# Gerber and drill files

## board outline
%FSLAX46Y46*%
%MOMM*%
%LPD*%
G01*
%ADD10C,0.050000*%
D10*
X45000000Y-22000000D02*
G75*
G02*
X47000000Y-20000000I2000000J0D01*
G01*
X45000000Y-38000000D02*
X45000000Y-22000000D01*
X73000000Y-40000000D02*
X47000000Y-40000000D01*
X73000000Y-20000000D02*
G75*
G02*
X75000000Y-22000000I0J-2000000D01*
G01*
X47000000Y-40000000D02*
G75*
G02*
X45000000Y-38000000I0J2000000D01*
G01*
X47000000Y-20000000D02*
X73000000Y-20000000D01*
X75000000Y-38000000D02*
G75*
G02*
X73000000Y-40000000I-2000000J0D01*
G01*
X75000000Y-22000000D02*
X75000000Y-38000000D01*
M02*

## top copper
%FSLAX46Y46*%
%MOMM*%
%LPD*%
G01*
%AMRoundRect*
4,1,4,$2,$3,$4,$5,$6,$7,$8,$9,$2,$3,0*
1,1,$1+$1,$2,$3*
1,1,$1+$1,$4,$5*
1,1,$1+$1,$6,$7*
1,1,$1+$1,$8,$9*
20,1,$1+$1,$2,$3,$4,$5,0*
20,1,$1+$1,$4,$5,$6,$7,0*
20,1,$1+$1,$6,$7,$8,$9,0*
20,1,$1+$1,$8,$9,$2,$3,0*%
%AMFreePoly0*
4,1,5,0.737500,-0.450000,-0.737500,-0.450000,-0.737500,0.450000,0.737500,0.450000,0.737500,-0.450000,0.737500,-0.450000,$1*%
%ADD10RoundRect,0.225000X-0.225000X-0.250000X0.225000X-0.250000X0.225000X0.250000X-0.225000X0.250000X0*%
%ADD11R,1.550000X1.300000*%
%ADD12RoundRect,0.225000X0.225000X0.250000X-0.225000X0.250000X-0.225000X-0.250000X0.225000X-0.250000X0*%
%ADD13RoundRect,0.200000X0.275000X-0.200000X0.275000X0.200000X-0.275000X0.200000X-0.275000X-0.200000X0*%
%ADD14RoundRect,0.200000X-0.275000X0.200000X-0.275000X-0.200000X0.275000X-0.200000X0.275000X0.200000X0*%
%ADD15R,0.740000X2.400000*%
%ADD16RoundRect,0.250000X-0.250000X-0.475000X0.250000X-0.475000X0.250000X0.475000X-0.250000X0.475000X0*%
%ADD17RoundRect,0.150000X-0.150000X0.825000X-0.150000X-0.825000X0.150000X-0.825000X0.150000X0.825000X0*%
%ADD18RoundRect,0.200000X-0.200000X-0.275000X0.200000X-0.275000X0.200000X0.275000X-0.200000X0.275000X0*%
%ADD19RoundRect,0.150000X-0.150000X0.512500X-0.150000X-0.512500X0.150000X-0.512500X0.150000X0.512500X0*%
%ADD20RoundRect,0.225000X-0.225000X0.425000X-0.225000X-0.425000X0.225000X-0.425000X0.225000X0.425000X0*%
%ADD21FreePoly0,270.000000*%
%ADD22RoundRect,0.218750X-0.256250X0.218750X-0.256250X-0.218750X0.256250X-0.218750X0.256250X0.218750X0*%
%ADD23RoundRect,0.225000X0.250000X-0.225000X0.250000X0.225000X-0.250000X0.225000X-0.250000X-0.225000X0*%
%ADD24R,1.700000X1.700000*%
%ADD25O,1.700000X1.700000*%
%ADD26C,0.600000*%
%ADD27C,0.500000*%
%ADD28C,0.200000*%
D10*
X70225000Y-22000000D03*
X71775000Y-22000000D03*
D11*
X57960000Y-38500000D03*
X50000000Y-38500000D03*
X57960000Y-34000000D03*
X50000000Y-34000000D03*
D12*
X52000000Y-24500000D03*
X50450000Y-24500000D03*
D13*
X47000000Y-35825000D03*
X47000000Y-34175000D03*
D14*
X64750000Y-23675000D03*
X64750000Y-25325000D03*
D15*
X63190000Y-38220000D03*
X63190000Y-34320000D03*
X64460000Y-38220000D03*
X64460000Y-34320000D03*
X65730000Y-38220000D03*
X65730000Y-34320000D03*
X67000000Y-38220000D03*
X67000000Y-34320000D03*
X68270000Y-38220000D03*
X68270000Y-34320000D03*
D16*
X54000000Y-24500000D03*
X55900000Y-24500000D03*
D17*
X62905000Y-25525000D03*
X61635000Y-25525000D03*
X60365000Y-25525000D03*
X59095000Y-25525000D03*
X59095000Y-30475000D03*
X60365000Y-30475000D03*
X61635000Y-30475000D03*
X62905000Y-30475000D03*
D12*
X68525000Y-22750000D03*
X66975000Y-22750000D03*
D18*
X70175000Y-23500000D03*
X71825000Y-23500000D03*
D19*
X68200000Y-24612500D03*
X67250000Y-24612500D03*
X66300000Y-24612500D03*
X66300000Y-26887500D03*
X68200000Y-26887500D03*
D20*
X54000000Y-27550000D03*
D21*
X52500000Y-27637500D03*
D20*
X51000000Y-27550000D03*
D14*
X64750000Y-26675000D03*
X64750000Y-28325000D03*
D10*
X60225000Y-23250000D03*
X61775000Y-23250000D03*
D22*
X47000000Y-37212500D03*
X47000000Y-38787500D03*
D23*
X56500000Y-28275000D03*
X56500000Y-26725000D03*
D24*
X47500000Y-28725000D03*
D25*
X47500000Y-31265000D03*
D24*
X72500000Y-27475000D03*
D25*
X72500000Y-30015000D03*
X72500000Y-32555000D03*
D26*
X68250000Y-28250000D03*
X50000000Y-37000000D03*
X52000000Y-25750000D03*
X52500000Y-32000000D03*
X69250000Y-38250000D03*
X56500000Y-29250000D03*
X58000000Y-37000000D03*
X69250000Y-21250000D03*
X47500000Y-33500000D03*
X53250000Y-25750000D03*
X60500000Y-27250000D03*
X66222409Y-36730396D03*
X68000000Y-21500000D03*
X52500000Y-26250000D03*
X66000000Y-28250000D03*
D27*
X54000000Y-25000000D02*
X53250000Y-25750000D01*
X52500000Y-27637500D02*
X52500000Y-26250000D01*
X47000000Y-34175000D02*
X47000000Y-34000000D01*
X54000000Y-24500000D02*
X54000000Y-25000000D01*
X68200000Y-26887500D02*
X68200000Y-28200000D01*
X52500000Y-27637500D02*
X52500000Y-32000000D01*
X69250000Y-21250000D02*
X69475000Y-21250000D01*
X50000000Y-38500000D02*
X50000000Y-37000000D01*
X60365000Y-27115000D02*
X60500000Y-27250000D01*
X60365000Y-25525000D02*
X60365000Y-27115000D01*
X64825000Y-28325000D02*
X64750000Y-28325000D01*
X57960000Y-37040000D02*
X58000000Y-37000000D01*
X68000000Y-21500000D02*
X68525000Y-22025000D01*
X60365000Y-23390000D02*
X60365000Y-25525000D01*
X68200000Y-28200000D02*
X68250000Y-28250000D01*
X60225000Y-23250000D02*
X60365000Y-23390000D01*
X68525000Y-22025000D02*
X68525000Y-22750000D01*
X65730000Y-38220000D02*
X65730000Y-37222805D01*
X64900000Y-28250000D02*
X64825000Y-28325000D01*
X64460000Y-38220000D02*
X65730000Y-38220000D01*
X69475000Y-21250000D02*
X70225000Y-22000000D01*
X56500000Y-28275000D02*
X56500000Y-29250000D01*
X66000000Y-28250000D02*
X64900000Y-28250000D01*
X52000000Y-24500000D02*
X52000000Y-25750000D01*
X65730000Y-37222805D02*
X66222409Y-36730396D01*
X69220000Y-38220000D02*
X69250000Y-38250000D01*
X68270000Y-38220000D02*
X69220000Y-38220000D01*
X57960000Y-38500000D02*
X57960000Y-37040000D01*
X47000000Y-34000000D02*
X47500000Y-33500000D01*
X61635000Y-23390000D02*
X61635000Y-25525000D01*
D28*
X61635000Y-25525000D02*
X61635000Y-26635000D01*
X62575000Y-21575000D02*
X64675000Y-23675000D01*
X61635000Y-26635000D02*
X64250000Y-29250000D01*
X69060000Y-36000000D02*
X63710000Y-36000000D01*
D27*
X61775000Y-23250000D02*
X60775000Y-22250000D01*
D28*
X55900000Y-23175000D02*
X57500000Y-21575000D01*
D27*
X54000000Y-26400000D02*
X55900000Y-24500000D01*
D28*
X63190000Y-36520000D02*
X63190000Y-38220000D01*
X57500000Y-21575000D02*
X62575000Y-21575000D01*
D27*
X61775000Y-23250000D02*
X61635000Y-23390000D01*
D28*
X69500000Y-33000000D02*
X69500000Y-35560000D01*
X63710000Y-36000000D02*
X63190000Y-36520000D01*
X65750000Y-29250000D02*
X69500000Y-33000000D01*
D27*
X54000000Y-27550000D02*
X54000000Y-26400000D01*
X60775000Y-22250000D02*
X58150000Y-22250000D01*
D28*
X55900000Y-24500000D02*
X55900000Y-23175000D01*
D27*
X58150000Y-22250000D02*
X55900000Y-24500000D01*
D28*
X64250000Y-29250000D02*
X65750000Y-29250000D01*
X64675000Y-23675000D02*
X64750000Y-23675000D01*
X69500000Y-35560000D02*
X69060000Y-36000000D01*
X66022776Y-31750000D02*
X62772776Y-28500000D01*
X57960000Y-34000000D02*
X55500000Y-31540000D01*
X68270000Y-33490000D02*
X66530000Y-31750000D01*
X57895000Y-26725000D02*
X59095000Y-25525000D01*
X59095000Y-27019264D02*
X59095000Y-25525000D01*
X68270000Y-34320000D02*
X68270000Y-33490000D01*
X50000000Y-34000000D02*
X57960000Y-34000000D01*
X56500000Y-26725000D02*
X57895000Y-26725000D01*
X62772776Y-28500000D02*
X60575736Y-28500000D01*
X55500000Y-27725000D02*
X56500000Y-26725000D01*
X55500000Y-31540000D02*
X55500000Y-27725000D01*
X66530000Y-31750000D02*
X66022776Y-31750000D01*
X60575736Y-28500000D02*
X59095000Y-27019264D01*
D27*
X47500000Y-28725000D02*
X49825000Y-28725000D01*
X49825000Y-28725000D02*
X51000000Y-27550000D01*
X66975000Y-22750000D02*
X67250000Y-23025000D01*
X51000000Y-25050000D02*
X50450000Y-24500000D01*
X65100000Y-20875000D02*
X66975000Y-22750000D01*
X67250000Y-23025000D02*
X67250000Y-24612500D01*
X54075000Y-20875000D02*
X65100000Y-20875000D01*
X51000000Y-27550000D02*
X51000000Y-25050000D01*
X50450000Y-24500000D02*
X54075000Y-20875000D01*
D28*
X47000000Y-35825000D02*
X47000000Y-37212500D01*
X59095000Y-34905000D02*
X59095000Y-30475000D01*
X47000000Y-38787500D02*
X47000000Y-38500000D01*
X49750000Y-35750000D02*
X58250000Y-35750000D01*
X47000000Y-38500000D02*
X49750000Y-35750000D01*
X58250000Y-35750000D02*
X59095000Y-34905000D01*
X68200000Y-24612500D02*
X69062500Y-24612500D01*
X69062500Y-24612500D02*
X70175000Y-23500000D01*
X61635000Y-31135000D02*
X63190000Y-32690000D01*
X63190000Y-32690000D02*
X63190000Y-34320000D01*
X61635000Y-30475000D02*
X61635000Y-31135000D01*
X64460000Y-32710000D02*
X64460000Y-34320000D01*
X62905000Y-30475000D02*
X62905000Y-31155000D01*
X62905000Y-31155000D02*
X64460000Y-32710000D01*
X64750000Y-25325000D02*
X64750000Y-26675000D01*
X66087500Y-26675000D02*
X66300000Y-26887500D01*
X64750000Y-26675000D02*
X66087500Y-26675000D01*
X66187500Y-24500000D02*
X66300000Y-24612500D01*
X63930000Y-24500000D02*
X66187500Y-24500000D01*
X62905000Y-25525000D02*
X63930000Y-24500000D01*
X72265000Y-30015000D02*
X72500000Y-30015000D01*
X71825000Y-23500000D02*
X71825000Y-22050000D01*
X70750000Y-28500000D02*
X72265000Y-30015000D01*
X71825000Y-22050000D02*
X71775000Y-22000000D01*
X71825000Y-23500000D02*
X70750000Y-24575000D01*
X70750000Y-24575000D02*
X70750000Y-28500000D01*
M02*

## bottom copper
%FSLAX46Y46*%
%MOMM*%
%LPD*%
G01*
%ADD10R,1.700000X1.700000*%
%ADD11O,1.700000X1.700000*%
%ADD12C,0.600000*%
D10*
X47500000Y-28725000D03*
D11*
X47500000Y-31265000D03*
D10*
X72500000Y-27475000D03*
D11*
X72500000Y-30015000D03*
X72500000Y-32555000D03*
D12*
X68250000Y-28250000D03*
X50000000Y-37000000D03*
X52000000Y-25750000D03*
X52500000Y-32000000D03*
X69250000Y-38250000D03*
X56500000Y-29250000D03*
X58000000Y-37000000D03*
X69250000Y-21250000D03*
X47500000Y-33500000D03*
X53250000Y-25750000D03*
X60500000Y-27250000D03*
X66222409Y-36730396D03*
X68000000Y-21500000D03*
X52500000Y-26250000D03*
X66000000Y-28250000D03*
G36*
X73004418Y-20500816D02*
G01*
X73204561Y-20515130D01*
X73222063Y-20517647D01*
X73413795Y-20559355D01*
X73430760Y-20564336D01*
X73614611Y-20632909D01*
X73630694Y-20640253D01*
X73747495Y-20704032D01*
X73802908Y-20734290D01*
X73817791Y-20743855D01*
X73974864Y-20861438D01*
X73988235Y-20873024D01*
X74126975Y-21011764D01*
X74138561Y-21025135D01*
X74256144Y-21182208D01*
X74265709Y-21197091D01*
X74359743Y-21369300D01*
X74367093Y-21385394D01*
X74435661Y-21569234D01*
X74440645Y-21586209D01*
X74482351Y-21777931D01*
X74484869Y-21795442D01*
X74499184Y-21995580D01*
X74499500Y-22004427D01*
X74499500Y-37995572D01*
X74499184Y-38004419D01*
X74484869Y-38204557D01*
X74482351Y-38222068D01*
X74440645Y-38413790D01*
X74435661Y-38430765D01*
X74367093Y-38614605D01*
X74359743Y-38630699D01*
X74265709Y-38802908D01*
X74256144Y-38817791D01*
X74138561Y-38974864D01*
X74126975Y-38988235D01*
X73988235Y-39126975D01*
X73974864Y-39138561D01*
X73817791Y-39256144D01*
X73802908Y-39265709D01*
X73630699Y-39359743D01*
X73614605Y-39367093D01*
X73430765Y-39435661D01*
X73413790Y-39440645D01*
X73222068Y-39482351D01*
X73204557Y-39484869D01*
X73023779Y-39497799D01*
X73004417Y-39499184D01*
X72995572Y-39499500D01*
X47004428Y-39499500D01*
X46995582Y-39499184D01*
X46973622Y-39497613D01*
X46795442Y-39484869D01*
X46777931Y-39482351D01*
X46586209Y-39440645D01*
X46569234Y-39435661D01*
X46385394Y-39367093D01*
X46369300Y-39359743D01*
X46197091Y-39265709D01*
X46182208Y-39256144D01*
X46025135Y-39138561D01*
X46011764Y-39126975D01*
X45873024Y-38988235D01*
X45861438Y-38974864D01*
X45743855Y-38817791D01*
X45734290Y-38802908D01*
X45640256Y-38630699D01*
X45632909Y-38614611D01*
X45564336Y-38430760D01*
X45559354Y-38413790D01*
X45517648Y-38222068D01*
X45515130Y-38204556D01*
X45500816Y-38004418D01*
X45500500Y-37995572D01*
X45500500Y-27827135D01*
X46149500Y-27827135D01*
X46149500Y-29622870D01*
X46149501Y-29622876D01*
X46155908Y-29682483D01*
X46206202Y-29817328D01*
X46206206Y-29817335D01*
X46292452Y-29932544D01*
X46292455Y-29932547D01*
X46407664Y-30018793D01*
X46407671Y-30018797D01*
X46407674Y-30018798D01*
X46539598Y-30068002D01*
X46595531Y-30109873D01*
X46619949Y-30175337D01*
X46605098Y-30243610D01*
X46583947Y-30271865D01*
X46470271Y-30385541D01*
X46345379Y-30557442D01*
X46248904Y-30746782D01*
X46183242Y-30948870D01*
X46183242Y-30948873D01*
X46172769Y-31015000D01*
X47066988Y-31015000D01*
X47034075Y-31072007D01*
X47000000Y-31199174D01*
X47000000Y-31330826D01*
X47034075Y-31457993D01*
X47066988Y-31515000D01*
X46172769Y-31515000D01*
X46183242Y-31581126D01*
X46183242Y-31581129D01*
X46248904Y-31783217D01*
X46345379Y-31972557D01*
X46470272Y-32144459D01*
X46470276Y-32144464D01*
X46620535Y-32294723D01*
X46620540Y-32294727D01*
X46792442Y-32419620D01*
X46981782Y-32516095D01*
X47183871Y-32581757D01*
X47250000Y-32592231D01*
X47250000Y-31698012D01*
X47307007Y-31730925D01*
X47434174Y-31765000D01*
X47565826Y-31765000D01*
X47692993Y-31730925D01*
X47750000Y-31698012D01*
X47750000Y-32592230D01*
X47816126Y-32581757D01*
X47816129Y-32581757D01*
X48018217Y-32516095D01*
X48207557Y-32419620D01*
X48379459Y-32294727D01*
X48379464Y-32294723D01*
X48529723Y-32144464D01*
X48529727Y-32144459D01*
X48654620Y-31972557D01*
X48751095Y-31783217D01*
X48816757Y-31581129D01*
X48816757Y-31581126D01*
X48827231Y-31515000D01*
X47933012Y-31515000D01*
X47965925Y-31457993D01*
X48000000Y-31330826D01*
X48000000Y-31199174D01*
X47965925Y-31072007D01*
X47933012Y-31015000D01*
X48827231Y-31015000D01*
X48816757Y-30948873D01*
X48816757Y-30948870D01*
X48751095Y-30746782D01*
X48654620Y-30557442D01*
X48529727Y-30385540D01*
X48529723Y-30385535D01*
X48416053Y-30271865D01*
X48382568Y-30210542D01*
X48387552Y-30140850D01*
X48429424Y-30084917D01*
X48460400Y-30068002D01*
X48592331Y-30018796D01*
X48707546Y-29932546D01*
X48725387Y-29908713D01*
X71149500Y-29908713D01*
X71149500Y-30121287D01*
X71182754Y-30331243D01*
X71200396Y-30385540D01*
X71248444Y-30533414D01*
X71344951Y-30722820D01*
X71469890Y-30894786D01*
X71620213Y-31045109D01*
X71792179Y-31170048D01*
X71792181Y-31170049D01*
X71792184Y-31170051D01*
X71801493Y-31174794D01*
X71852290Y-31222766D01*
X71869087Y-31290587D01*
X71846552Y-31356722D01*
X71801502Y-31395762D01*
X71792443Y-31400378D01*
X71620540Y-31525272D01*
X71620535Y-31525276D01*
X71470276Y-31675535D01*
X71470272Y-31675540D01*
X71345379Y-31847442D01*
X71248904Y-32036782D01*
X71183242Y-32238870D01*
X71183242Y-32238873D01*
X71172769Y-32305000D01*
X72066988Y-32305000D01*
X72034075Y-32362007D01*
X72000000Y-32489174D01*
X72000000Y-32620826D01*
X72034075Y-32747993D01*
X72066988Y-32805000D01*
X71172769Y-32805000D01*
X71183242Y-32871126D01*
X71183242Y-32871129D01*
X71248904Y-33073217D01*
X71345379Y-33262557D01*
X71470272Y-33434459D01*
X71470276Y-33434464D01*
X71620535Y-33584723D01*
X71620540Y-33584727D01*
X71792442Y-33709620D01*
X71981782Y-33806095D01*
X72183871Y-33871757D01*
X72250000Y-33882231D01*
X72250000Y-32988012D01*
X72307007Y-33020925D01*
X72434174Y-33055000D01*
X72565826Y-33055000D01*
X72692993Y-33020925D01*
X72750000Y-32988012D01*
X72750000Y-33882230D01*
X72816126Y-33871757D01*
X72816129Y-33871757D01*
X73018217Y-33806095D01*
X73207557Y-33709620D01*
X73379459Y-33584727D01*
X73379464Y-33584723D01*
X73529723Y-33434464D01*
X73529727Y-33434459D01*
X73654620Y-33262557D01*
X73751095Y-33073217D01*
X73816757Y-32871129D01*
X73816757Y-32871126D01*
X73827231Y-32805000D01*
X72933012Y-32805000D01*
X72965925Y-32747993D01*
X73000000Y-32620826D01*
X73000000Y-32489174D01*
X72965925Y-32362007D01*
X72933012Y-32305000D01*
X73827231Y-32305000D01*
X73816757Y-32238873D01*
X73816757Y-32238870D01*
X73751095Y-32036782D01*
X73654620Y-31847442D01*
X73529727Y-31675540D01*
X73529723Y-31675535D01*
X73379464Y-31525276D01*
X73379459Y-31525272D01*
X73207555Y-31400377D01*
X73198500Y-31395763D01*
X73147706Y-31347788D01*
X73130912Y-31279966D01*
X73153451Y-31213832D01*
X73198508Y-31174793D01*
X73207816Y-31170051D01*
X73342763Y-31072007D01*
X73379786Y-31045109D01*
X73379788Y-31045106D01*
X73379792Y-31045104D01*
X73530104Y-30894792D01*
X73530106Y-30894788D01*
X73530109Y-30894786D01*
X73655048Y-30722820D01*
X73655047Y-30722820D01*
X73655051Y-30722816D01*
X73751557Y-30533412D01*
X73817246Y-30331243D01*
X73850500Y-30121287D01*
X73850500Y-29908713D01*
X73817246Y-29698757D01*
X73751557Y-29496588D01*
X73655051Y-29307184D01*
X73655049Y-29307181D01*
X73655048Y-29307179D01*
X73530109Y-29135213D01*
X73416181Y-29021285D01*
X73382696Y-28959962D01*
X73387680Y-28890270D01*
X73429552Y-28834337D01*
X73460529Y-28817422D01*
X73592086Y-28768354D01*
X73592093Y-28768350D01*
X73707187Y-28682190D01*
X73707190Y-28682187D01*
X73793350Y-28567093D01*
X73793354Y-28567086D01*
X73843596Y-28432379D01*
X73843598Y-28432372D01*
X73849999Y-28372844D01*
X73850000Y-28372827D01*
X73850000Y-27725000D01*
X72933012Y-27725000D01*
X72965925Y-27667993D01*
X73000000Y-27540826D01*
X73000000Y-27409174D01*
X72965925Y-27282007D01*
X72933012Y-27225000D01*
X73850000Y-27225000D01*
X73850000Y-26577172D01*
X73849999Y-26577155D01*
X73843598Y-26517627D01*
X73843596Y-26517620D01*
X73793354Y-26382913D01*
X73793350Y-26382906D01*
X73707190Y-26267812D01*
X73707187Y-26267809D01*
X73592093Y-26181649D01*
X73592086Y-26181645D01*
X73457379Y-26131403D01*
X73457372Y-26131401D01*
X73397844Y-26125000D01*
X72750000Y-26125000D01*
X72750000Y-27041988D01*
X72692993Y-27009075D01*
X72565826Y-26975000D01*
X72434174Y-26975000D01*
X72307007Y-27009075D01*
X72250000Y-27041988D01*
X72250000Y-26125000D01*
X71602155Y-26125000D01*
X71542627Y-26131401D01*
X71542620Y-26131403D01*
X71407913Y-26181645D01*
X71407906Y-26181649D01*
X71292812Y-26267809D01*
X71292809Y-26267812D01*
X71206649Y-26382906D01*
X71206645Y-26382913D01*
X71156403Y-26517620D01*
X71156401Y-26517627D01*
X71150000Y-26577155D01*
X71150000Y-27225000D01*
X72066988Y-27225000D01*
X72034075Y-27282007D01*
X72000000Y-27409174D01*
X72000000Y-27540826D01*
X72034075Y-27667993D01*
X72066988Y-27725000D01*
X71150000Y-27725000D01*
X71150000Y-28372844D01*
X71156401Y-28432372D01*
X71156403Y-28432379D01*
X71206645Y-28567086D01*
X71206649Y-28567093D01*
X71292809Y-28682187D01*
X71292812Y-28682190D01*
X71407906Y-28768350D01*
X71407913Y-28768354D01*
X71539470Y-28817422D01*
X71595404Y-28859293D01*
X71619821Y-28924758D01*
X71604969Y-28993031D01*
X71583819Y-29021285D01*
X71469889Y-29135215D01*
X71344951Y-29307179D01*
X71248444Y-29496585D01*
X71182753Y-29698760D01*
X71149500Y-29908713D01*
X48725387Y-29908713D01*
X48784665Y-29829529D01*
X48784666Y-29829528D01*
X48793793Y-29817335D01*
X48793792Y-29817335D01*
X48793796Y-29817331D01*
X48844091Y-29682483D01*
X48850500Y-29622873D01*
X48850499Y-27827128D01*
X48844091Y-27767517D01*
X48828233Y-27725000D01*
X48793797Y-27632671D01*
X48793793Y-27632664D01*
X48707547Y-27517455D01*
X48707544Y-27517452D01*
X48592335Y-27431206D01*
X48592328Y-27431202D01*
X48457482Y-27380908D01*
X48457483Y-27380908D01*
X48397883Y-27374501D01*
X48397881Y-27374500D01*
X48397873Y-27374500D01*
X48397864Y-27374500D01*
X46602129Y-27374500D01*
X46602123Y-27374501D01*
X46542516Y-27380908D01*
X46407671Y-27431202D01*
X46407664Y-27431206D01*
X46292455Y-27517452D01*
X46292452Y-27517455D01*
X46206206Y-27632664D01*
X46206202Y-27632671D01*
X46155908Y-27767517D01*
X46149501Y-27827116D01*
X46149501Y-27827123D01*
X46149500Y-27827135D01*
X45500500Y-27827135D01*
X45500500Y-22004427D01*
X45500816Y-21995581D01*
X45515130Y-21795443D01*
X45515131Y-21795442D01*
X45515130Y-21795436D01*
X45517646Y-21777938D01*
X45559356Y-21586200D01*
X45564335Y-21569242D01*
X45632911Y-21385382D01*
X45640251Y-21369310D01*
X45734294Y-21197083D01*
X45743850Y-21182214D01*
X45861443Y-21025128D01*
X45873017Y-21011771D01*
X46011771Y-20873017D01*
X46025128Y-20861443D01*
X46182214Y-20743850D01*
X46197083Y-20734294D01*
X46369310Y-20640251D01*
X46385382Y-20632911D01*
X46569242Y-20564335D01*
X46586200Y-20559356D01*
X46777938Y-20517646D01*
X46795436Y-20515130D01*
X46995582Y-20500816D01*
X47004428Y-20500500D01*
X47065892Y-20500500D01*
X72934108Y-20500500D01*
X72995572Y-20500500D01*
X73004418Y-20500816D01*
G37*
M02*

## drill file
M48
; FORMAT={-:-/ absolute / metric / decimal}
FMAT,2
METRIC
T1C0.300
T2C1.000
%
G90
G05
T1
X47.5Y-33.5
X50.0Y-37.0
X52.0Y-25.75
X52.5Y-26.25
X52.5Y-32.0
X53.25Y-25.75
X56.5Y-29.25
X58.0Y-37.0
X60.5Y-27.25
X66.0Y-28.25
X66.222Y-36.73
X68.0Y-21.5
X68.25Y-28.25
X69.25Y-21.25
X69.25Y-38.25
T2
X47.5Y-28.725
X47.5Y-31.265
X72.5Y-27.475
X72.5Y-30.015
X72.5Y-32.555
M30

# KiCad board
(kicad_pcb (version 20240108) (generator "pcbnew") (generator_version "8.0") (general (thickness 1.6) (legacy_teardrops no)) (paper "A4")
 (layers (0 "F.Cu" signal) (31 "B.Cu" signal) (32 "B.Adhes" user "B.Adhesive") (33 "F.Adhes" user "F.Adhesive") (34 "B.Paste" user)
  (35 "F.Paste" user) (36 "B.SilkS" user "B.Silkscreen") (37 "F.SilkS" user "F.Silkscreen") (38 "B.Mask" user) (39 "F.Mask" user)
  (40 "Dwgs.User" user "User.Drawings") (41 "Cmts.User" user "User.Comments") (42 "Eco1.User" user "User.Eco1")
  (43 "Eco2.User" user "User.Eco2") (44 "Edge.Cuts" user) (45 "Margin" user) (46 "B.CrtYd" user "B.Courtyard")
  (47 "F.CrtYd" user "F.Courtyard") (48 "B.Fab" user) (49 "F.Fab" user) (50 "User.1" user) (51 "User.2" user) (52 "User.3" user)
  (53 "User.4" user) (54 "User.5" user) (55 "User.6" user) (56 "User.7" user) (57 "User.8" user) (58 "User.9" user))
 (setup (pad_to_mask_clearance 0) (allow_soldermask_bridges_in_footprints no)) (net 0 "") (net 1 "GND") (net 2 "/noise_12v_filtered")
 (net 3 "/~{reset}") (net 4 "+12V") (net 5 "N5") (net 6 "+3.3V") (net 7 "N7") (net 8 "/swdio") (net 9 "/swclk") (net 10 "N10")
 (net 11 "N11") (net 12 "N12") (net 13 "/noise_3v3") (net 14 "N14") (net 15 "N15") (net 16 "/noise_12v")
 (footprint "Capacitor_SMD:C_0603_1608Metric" (layer "F.Cu") (at 71 22)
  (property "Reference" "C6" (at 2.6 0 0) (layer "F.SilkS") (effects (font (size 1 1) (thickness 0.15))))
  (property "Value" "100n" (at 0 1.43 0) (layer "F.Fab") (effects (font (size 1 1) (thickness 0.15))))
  (pad "1" smd roundrect (at -0.775 0) (size 0.9 0.95) (layers "F.Cu") (roundrect_rratio 0.25) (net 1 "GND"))
  (pad "2" smd roundrect (at 0.775 0) (size 0.9 0.95) (layers "F.Cu") (roundrect_rratio 0.25) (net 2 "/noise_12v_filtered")))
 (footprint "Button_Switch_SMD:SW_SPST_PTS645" (layer "F.Cu") (at 53.98 36.25 180)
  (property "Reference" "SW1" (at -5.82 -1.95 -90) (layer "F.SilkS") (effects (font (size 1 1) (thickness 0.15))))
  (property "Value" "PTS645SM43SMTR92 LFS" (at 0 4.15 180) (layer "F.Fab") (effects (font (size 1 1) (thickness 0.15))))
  (pad "1" smd rect (at -3.98 -2.25 180) (size 1.55 1.3) (layers "F.Cu") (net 1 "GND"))
  (pad "1" smd rect (at 3.98 -2.25 180) (size 1.55 1.3) (layers "F.Cu") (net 1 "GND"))
  (pad "2" smd rect (at -3.98 2.25 180) (size 1.55 1.3) (layers "F.Cu") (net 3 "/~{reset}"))
  (pad "2" smd rect (at 3.98 2.25 180) (size 1.55 1.3) (layers "F.Cu") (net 3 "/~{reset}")))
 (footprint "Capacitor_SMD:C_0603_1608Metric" (layer "F.Cu") (at 51.225 24.5 180)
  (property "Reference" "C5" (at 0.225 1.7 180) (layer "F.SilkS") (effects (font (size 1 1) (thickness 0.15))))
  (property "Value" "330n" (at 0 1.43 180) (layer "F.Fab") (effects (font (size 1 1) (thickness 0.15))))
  (pad "1" smd roundrect (at -0.775 0 180) (size 0.9 0.95) (layers "F.Cu") (roundrect_rratio 0.25) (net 1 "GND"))
  (pad "2" smd roundrect (at 0.775 0 180) (size 0.9 0.95) (layers "F.Cu") (roundrect_rratio 0.25) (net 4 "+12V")))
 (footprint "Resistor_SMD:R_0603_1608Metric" (layer "F.Cu") (at 47 35 90)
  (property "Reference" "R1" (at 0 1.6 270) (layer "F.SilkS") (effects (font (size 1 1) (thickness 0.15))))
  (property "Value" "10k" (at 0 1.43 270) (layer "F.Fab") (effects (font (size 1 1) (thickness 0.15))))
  (pad "1" smd roundrect (at -0.825 0 90) (size 0.8 0.95) (layers "F.Cu") (roundrect_rratio 0.25) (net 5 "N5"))
  (pad "2" smd roundrect (at 0.825 0 90) (size 0.8 0.95) (layers "F.Cu") (roundrect_rratio 0.25) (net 1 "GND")))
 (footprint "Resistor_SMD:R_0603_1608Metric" (layer "F.Cu") (at 64.75 24.5 -90)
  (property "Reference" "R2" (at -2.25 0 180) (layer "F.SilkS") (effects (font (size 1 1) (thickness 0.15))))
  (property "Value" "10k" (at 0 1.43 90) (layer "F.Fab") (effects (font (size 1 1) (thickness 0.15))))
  (pad "1" smd roundrect (at -0.825 0 270) (size 0.8 0.95) (layers "F.Cu") (roundrect_rratio 0.25) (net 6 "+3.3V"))
  (pad "2" smd roundrect (at 0.825 0 270) (size 0.8 0.95) (layers "F.Cu") (roundrect_rratio 0.25) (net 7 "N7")))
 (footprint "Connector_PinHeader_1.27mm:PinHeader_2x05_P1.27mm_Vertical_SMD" (layer "F.Cu") (at 65.73 36.27 90)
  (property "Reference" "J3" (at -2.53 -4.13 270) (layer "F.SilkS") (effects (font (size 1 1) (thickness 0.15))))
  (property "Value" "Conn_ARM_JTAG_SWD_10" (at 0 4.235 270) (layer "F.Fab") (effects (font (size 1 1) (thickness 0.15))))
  (pad "1" smd rect (at -1.95 -2.54 90) (size 2.4 0.74) (layers "F.Cu") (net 6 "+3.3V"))
  (pad "2" smd rect (at 1.95 -2.54 90) (size 2.4 0.74) (layers "F.Cu") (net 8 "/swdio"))
  (pad "3" smd rect (at -1.95 -1.27 90) (size 2.4 0.74) (layers "F.Cu") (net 1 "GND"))
  (pad "4" smd rect (at 1.95 -1.27 90) (size 2.4 0.74) (layers "F.Cu") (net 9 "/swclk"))
  (pad "5" smd rect (at -1.95 0 90) (size 2.4 0.74) (layers "F.Cu") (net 1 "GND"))
  (pad "6" smd rect (at 1.95 0 90) (size 2.4 0.74) (layers "F.Cu") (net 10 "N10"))
  (pad "7" smd rect (at -1.95 1.27 90) (size 2.4 0.74) (layers "F.Cu") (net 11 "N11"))
  (pad "8" smd rect (at 1.95 1.27 90) (size 2.4 0.74) (layers "F.Cu") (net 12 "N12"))
  (pad "9" smd rect (at -1.95 2.54 90) (size 2.4 0.74) (layers "F.Cu") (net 1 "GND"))
  (pad "10" smd rect (at 1.95 2.54 90) (size 2.4 0.74) (layers "F.Cu") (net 3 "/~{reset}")))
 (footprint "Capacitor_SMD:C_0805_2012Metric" (layer "F.Cu") (at 54.95 24.5)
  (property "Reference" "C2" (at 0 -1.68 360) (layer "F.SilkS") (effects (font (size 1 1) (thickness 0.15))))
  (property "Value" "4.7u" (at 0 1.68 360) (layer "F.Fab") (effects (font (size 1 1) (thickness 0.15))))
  (pad "1" smd roundrect (at -0.95 0) (size 1 1.45) (layers "F.Cu") (roundrect_rratio 0.25) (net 1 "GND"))
  (pad "2" smd roundrect (at 0.95 0) (size 1 1.45) (layers "F.Cu") (roundrect_rratio 0.25) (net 6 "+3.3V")))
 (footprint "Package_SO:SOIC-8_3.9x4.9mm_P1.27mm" (layer "F.Cu") (at 61 28 -90)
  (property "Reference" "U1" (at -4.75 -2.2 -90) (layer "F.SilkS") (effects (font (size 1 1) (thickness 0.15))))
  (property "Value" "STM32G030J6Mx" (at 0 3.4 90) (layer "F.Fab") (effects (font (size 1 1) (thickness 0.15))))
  (pad "1" smd roundrect (at -2.475 -1.905 270) (size 1.95 0.6) (layers "F.Cu") (roundrect_rratio 0.25) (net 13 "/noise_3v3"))
  (pad "2" smd roundrect (at -2.475 -0.635 270) (size 1.95 0.6) (layers "F.Cu") (roundrect_rratio 0.25) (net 6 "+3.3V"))
  (pad "3" smd roundrect (at -2.475 0.635 270) (size 1.95 0.6) (layers "F.Cu") (roundrect_rratio 0.25) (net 1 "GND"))
  (pad "4" smd roundrect (at -2.475 1.905 270) (size 1.95 0.6) (layers "F.Cu") (roundrect_rratio 0.25) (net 3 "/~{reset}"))
  (pad "5" smd roundrect (at 2.475 1.905 270) (size 1.95 0.6) (layers "F.Cu") (roundrect_rratio 0.25) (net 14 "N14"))
  (pad "6" smd roundrect (at 2.475 0.635 270) (size 1.95 0.6) (layers "F.Cu") (roundrect_rratio 0.25) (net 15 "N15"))
  (pad "7" smd roundrect (at 2.475 -0.635 270) (size 1.95 0.6) (layers "F.Cu") (roundrect_rratio 0.25) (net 8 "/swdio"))
  (pad "8" smd roundrect (at 2.475 -1.905 270) (size 1.95 0.6) (layers "F.Cu") (roundrect_rratio 0.25) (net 9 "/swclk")))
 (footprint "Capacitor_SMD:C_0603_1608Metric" (layer "F.Cu") (at 67.75 22.75 180)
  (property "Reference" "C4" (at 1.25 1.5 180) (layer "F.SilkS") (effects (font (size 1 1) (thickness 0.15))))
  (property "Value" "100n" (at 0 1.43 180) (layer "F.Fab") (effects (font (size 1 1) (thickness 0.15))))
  (pad "1" smd roundrect (at -0.775 0 180) (size 0.9 0.95) (layers "F.Cu") (roundrect_rratio 0.25) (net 1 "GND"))
  (pad "2" smd roundrect (at 0.775 0 180) (size 0.9 0.95) (layers "F.Cu") (roundrect_rratio 0.25) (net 4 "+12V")))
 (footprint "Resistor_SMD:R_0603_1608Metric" (layer "F.Cu") (at 71 23.5)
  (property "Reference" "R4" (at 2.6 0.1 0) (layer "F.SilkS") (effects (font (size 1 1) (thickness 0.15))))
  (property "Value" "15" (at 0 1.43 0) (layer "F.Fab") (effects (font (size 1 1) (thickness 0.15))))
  (pad "1" smd roundrect (at -0.825 0) (size 0.8 0.95) (layers "F.Cu") (roundrect_rratio 0.25) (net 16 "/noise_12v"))
  (pad "2" smd roundrect (at 0.825 0) (size 0.8 0.95) (layers "F.Cu") (roundrect_rratio 0.25) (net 2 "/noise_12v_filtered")))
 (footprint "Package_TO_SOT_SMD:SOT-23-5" (layer "F.Cu") (at 67.25 25.75 -90)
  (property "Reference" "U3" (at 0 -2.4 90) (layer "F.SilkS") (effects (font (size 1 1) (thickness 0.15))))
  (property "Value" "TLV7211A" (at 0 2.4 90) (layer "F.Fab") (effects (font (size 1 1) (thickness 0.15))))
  (pad "1" smd roundrect (at -1.1375 -0.95 270) (size 1.325 0.6) (layers "F.Cu") (roundrect_rratio 0.25) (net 16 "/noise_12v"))
  (pad "2" smd roundrect (at -1.1375 0 270) (size 1.325 0.6) (layers "F.Cu") (roundrect_rratio 0.25) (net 4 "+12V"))
  (pad "3" smd roundrect (at -1.1375 0.95 270) (size 1.325 0.6) (layers "F.Cu") (roundrect_rratio 0.25) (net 13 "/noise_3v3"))
  (pad "4" smd roundrect (at 1.1375 0.95 270) (size 1.325 0.6) (layers "F.Cu") (roundrect_rratio 0.25) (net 7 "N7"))
  (pad "5" smd roundrect (at 1.1375 -0.95 270) (size 1.325 0.6) (layers "F.Cu") (roundrect_rratio 0.25) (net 1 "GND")))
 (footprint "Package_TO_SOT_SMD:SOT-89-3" (layer "F.Cu") (at 52.5 29.5 -90)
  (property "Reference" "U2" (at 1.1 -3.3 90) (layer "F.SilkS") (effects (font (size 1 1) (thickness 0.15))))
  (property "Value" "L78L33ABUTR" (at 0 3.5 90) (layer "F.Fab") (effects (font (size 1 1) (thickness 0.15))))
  (pad "1" smd roundrect (at -1.95 -1.5 270) (size 1.3 0.9) (layers "F.Cu") (roundrect_rratio 0.25) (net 6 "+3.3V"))
  (pad "2" smd custom (at -1.8625 0 270) (size 1.475 0.9) (layers "F.Cu") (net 1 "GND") (zone_connect 2) (thermal_bridge_angle 45)
   (options (clearance outline) (anchor rect)) (primitives))
  (pad "3" smd roundrect (at -1.95 1.5 270) (size 1.3 0.9) (layers "F.Cu") (roundrect_rratio 0.25) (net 4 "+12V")))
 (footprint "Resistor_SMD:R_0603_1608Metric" (layer "F.Cu") (at 64.75 27.5 -90)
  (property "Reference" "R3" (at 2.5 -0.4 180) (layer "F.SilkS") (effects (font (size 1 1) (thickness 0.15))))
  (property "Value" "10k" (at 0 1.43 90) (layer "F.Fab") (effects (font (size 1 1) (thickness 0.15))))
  (pad "1" smd roundrect (at -0.825 0 270) (size 0.8 0.95) (layers "F.Cu") (roundrect_rratio 0.25) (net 7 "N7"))
  (pad "2" smd roundrect (at 0.825 0 270) (size 0.8 0.95) (layers "F.Cu") (roundrect_rratio 0.25) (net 1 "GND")))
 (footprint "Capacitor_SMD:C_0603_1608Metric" (layer "F.Cu") (at 61 23.25)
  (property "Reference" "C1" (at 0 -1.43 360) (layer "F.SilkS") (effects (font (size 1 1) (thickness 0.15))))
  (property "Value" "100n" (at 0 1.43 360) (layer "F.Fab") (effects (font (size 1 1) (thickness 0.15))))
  (pad "1" smd roundrect (at -0.775 0) (size 0.9 0.95) (layers "F.Cu") (roundrect_rratio 0.25) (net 1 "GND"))
  (pad "2" smd roundrect (at 0.775 0) (size 0.9 0.95) (layers "F.Cu") (roundrect_rratio 0.25) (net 6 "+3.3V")))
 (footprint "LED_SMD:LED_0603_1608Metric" (layer "F.Cu") (at 47 38 -90)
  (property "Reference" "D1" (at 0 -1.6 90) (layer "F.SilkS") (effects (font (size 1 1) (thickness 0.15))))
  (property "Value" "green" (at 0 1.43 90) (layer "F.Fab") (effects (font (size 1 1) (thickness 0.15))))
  (pad "1" smd roundrect (at -0.7875 0 270) (size 0.875 0.95) (layers "F.Cu") (roundrect_rratio 0.25) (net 5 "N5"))
  (pad "2" smd roundrect (at 0.7875 0 270) (size 0.875 0.95) (layers "F.Cu") (roundrect_rratio 0.25) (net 14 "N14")))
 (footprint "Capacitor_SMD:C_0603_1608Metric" (layer "F.Cu") (at 56.5 27.5 90)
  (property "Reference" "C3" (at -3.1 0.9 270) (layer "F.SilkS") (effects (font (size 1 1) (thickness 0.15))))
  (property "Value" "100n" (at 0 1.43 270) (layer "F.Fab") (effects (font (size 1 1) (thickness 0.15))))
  (pad "1" smd roundrect (at -0.775 0 90) (size 0.9 0.95) (layers "F.Cu") (roundrect_rratio 0.25) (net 1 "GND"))
  (pad "2" smd roundrect (at 0.775 0 90) (size 0.9 0.95) (layers "F.Cu") (roundrect_rratio 0.25) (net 3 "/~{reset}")))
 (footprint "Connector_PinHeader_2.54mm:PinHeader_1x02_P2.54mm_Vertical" (layer "B.Cu") (at 47.5 28.725 180)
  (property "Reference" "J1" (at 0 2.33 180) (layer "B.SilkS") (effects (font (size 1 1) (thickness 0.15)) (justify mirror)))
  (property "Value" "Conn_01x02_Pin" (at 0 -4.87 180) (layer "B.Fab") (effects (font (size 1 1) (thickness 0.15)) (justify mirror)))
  (pad "1" thru_hole rect (at 0 0 180) (size 1.7 1.7) (drill 1) (layers "*.Cu" "*.Mask") (remove_unused_layers no) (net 4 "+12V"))
  (pad "2" thru_hole oval (at 0 -2.54 180) (size 1.7 1.7) (drill 1) (layers "*.Cu" "*.Mask") (remove_unused_layers no) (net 1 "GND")))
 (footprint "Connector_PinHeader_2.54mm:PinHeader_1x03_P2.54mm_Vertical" (layer "B.Cu") (at 72.5 27.475 180)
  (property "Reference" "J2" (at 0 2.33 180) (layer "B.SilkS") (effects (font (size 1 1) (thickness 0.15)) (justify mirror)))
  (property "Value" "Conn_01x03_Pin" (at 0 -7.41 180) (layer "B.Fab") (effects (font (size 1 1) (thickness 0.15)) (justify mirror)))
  (pad "1" thru_hole rect (at 0 0 180) (size 1.7 1.7) (drill 1) (layers "*.Cu" "*.Mask") (remove_unused_layers no) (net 1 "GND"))
  (pad "2" thru_hole oval (at 0 -2.54 180) (size 1.7 1.7) (drill 1) (layers "*.Cu" "*.Mask") (remove_unused_layers no)
   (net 2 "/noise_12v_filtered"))
  (pad "3" thru_hole oval (at 0 -5.08 180) (size 1.7 1.7) (drill 1) (layers "*.Cu" "*.Mask") (remove_unused_layers no) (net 1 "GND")))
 (gr_arc (start 45 22) (mid 45.585786 20.585786) (end 47 20) (stroke (width 0.05) (type default)) (layer "Edge.Cuts"))
 (gr_line (start 45 38) (end 45 22) (stroke (width 0.05) (type default)) (layer "Edge.Cuts"))
 (gr_line (start 73 40) (end 47 40) (stroke (width 0.05) (type default)) (layer "Edge.Cuts"))
 (gr_arc (start 73 20) (mid 74.414214 20.585786) (end 75 22) (stroke (width 0.05) (type default)) (layer "Edge.Cuts"))
 (gr_arc (start 47 40) (mid 45.585786 39.414214) (end 45 38) (stroke (width 0.05) (type default)) (layer "Edge.Cuts"))
 (gr_line (start 47 20) (end 73 20) (stroke (width 0.05) (type default)) (layer "Edge.Cuts"))
 (gr_arc (start 75 38) (mid 74.414214 39.414214) (end 73 40) (stroke (width 0.05) (type default)) (layer "Edge.Cuts"))
 (gr_line (start 75 22) (end 75 38) (stroke (width 0.05) (type default)) (layer "Edge.Cuts"))
 (segment (start 54 25) (end 53.25 25.75) (width 0.5) (layer "F.Cu") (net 1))
 (segment (start 52.5 27.6375) (end 52.5 26.25) (width 0.5) (layer "F.Cu") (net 1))
 (segment (start 47 34.175) (end 47 34) (width 0.5) (layer "F.Cu") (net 1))
 (segment (start 54 24.5) (end 54 25) (width 0.5) (layer "F.Cu") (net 1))
 (segment (start 68.2 26.8875) (end 68.2 28.2) (width 0.5) (layer "F.Cu") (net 1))
 (segment (start 52.5 27.6375) (end 52.5 32) (width 0.5) (layer "F.Cu") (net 1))
 (segment (start 69.25 21.25) (end 69.475 21.25) (width 0.5) (layer "F.Cu") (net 1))
 (segment (start 50 38.5) (end 50 37) (width 0.5) (layer "F.Cu") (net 1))
 (segment (start 60.365 27.115) (end 60.5 27.25) (width 0.5) (layer "F.Cu") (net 1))
 (segment (start 60.365 25.525) (end 60.365 27.115) (width 0.5) (layer "F.Cu") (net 1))
 (segment (start 64.825 28.325) (end 64.75 28.325) (width 0.5) (layer "F.Cu") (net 1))
 (segment (start 57.96 37.04) (end 58 37) (width 0.5) (layer "F.Cu") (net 1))
 (segment (start 68 21.5) (end 68.525 22.025) (width 0.5) (layer "F.Cu") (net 1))
 (segment (start 60.365 23.39) (end 60.365 25.525) (width 0.5) (layer "F.Cu") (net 1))
 (segment (start 68.2 28.2) (end 68.25 28.25) (width 0.5) (layer "F.Cu") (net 1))
 (segment (start 60.225 23.25) (end 60.365 23.39) (width 0.5) (layer "F.Cu") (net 1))
 (segment (start 68.525 22.025) (end 68.525 22.75) (width 0.5) (layer "F.Cu") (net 1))
 (segment (start 65.73 38.22) (end 65.73 37.222805) (width 0.5) (layer "F.Cu") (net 1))
 (segment (start 64.9 28.25) (end 64.825 28.325) (width 0.5) (layer "F.Cu") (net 1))
 (segment (start 64.46 38.22) (end 65.73 38.22) (width 0.5) (layer "F.Cu") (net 1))
 (segment (start 69.475 21.25) (end 70.225 22) (width 0.5) (layer "F.Cu") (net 1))
 (segment (start 56.5 28.275) (end 56.5 29.25) (width 0.5) (layer "F.Cu") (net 1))
 (segment (start 66 28.25) (end 64.9 28.25) (width 0.5) (layer "F.Cu") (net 1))
 (segment (start 52 24.5) (end 52 25.75) (width 0.5) (layer "F.Cu") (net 1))
 (segment (start 65.73 37.222805) (end 66.222409 36.730396) (width 0.5) (layer "F.Cu") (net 1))
 (segment (start 69.22 38.22) (end 69.25 38.25) (width 0.5) (layer "F.Cu") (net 1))
 (segment (start 68.27 38.22) (end 69.22 38.22) (width 0.5) (layer "F.Cu") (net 1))
 (segment (start 57.96 38.5) (end 57.96 37.04) (width 0.5) (layer "F.Cu") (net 1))
 (segment (start 47 34) (end 47.5 33.5) (width 0.5) (layer "F.Cu") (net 1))
 (via (at 68.25 28.25) (size 0.6) (drill 0.3) (layers "F.Cu" "B.Cu") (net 1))
 (via (at 50 37) (size 0.6) (drill 0.3) (layers "F.Cu" "B.Cu") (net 1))
 (via (at 52 25.75) (size 0.6) (drill 0.3) (layers "F.Cu" "B.Cu") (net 1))
 (via (at 52.5 32) (size 0.6) (drill 0.3) (layers "F.Cu" "B.Cu") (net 1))
 (via (at 69.25 38.25) (size 0.6) (drill 0.3) (layers "F.Cu" "B.Cu") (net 1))
 (via (at 56.5 29.25) (size 0.6) (drill 0.3) (layers "F.Cu" "B.Cu") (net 1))
 (via (at 58 37) (size 0.6) (drill 0.3) (layers "F.Cu" "B.Cu") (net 1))
 (via (at 69.25 21.25) (size 0.6) (drill 0.3) (layers "F.Cu" "B.Cu") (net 1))
 (via (at 47.5 33.5) (size 0.6) (drill 0.3) (layers "F.Cu" "B.Cu") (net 1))
 (via (at 53.25 25.75) (size 0.6) (drill 0.3) (layers "F.Cu" "B.Cu") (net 1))
 (via (at 60.5 27.25) (size 0.6) (drill 0.3) (layers "F.Cu" "B.Cu") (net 1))
 (via (at 66.222409 36.730396) (size 0.6) (drill 0.3) (layers "F.Cu" "B.Cu") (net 1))
 (via (at 68 21.5) (size 0.6) (drill 0.3) (layers "F.Cu" "B.Cu") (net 1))
 (via (at 52.5 26.25) (size 0.6) (drill 0.3) (layers "F.Cu" "B.Cu") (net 1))
 (via (at 66 28.25) (size 0.6) (drill 0.3) (layers "F.Cu" "B.Cu") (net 1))
 (segment (start 61.635 23.39) (end 61.635 25.525) (width 0.5) (layer "F.Cu") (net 6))
 (segment (start 61.635 25.525) (end 61.635 26.635) (width 0.2) (layer "F.Cu") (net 6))
 (segment (start 62.575 21.575) (end 64.675 23.675) (width 0.2) (layer "F.Cu") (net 6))
 (segment (start 61.635 26.635) (end 64.25 29.25) (width 0.2) (layer "F.Cu") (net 6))
 (segment (start 69.06 36) (end 63.71 36) (width 0.2) (layer "F.Cu") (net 6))
 (segment (start 61.775 23.25) (end 60.775 22.25) (width 0.5) (layer "F.Cu") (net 6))
 (segment (start 55.9 23.175) (end 57.5 21.575) (width 0.2) (layer "F.Cu") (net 6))
 (segment (start 54 26.4) (end 55.9 24.5) (width 0.5) (layer "F.Cu") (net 6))
 (segment (start 63.19 36.52) (end 63.19 38.22) (width 0.2) (layer "F.Cu") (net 6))
 (segment (start 57.5 21.575) (end 62.575 21.575) (width 0.2) (layer "F.Cu") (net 6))
 (segment (start 61.775 23.25) (end 61.635 23.39) (width 0.5) (layer "F.Cu") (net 6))
 (segment (start 69.5 33) (end 69.5 35.56) (width 0.2) (layer "F.Cu") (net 6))
 (segment (start 63.71 36) (end 63.19 36.52) (width 0.2) (layer "F.Cu") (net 6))
 (segment (start 65.75 29.25) (end 69.5 33) (width 0.2) (layer "F.Cu") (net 6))
 (segment (start 54 27.55) (end 54 26.4) (width 0.5) (layer "F.Cu") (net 6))
 (segment (start 60.775 22.25) (end 58.15 22.25) (width 0.5) (layer "F.Cu") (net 6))
 (segment (start 55.9 24.5) (end 55.9 23.175) (width 0.2) (layer "F.Cu") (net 6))
 (segment (start 58.15 22.25) (end 55.9 24.5) (width 0.5) (layer "F.Cu") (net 6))
 (segment (start 64.25 29.25) (end 65.75 29.25) (width 0.2) (layer "F.Cu") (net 6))
 (segment (start 64.675 23.675) (end 64.75 23.675) (width 0.2) (layer "F.Cu") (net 6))
 (segment (start 69.5 35.56) (end 69.06 36) (width 0.2) (layer "F.Cu") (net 6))
 (segment (start 66.022776 31.75) (end 62.772776 28.5) (width 0.2) (layer "F.Cu") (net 3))
 (segment (start 57.96 34) (end 55.5 31.54) (width 0.2) (layer "F.Cu") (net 3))
 (segment (start 68.27 33.49) (end 66.53 31.75) (width 0.2) (layer "F.Cu") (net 3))
 (segment (start 57.895 26.725) (end 59.095 25.525) (width 0.2) (layer "F.Cu") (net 3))
 (segment (start 59.095 27.019264) (end 59.095 25.525) (width 0.2) (layer "F.Cu") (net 3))
 (segment (start 68.27 34.32) (end 68.27 33.49) (width 0.2) (layer "F.Cu") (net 3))
 (segment (start 50 34) (end 57.96 34) (width 0.2) (layer "F.Cu") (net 3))
 (segment (start 56.5 26.725) (end 57.895 26.725) (width 0.2) (layer "F.Cu") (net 3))
 (segment (start 62.772776 28.5) (end 60.575736 28.5) (width 0.2) (layer "F.Cu") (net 3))
 (segment (start 55.5 27.725) (end 56.5 26.725) (width 0.2) (layer "F.Cu") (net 3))
 (segment (start 55.5 31.54) (end 55.5 27.725) (width 0.2) (layer "F.Cu") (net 3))
 (segment (start 66.53 31.75) (end 66.022776 31.75) (width 0.2) (layer "F.Cu") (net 3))
 (segment (start 60.575736 28.5) (end 59.095 27.019264) (width 0.2) (layer "F.Cu") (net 3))
 (segment (start 47.5 28.725) (end 49.825 28.725) (width 0.5) (layer "F.Cu") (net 4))
 (segment (start 49.825 28.725) (end 51 27.55) (width 0.5) (layer "F.Cu") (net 4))
 (segment (start 66.975 22.75) (end 67.25 23.025) (width 0.5) (layer "F.Cu") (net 4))
 (segment (start 51 25.05) (end 50.45 24.5) (width 0.5) (layer "F.Cu") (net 4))
 (segment (start 65.1 20.875) (end 66.975 22.75) (width 0.5) (layer "F.Cu") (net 4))
 (segment (start 67.25 23.025) (end 67.25 24.6125) (width 0.5) (layer "F.Cu") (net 4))
 (segment (start 54.075 20.875) (end 65.1 20.875) (width 0.5) (layer "F.Cu") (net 4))
 (segment (start 51 27.55) (end 51 25.05) (width 0.5) (layer "F.Cu") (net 4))
 (segment (start 50.45 24.5) (end 54.075 20.875) (width 0.5) (layer "F.Cu") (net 4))
 (segment (start 47 35.825) (end 47 37.2125) (width 0.2) (layer "F.Cu") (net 5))
 (segment (start 59.095 34.905) (end 59.095 30.475) (width 0.2) (layer "F.Cu") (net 14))
 (segment (start 47 38.7875) (end 47 38.5) (width 0.2) (layer "F.Cu") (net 14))
 (segment (start 49.75 35.75) (end 58.25 35.75) (width 0.2) (layer "F.Cu") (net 14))
 (segment (start 47 38.5) (end 49.75 35.75) (width 0.2) (layer "F.Cu") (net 14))
 (segment (start 58.25 35.75) (end 59.095 34.905) (width 0.2) (layer "F.Cu") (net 14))
 (segment (start 68.2 24.6125) (end 69.0625 24.6125) (width 0.2) (layer "F.Cu") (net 16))
 (segment (start 69.0625 24.6125) (end 70.175 23.5) (width 0.2) (layer "F.Cu") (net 16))
 (segment (start 61.635 31.135) (end 63.19 32.69) (width 0.2) (layer "F.Cu") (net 8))
 (segment (start 63.19 32.69) (end 63.19 34.32) (width 0.2) (layer "F.Cu") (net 8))
 (segment (start 61.635 30.475) (end 61.635 31.135) (width 0.2) (layer "F.Cu") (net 8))
 (segment (start 64.46 32.71) (end 64.46 34.32) (width 0.2) (layer "F.Cu") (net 9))
 (segment (start 62.905 30.475) (end 62.905 31.155) (width 0.2) (layer "F.Cu") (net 9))
 (segment (start 62.905 31.155) (end 64.46 32.71) (width 0.2) (layer "F.Cu") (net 9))
 (segment (start 64.75 25.325) (end 64.75 26.675) (width 0.2) (layer "F.Cu") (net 7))
 (segment (start 66.0875 26.675) (end 66.3 26.8875) (width 0.2) (layer "F.Cu") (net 7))
 (segment (start 64.75 26.675) (end 66.0875 26.675) (width 0.2) (layer "F.Cu") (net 7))
 (segment (start 66.1875 24.5) (end 66.3 24.6125) (width 0.2) (layer "F.Cu") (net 13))
 (segment (start 63.93 24.5) (end 66.1875 24.5) (width 0.2) (layer "F.Cu") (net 13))
 (segment (start 62.905 25.525) (end 63.93 24.5) (width 0.2) (layer "F.Cu") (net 13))
 (segment (start 72.265 30.015) (end 72.5 30.015) (width 0.2) (layer "F.Cu") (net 2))
 (segment (start 71.825 23.5) (end 71.825 22.05) (width 0.2) (layer "F.Cu") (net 2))
 (segment (start 70.75 28.5) (end 72.265 30.015) (width 0.2) (layer "F.Cu") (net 2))
 (segment (start 71.825 22.05) (end 71.775 22) (width 0.2) (layer "F.Cu") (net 2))
 (segment (start 71.825 23.5) (end 70.75 24.575) (width 0.2) (layer "F.Cu") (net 2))
 (segment (start 70.75 24.575) (end 70.75 28.5) (width 0.2) (layer "F.Cu") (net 2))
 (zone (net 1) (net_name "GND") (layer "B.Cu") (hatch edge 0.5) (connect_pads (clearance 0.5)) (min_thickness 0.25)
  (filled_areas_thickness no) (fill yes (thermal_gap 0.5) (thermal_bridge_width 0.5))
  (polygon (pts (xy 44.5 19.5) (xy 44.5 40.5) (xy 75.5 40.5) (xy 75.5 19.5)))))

